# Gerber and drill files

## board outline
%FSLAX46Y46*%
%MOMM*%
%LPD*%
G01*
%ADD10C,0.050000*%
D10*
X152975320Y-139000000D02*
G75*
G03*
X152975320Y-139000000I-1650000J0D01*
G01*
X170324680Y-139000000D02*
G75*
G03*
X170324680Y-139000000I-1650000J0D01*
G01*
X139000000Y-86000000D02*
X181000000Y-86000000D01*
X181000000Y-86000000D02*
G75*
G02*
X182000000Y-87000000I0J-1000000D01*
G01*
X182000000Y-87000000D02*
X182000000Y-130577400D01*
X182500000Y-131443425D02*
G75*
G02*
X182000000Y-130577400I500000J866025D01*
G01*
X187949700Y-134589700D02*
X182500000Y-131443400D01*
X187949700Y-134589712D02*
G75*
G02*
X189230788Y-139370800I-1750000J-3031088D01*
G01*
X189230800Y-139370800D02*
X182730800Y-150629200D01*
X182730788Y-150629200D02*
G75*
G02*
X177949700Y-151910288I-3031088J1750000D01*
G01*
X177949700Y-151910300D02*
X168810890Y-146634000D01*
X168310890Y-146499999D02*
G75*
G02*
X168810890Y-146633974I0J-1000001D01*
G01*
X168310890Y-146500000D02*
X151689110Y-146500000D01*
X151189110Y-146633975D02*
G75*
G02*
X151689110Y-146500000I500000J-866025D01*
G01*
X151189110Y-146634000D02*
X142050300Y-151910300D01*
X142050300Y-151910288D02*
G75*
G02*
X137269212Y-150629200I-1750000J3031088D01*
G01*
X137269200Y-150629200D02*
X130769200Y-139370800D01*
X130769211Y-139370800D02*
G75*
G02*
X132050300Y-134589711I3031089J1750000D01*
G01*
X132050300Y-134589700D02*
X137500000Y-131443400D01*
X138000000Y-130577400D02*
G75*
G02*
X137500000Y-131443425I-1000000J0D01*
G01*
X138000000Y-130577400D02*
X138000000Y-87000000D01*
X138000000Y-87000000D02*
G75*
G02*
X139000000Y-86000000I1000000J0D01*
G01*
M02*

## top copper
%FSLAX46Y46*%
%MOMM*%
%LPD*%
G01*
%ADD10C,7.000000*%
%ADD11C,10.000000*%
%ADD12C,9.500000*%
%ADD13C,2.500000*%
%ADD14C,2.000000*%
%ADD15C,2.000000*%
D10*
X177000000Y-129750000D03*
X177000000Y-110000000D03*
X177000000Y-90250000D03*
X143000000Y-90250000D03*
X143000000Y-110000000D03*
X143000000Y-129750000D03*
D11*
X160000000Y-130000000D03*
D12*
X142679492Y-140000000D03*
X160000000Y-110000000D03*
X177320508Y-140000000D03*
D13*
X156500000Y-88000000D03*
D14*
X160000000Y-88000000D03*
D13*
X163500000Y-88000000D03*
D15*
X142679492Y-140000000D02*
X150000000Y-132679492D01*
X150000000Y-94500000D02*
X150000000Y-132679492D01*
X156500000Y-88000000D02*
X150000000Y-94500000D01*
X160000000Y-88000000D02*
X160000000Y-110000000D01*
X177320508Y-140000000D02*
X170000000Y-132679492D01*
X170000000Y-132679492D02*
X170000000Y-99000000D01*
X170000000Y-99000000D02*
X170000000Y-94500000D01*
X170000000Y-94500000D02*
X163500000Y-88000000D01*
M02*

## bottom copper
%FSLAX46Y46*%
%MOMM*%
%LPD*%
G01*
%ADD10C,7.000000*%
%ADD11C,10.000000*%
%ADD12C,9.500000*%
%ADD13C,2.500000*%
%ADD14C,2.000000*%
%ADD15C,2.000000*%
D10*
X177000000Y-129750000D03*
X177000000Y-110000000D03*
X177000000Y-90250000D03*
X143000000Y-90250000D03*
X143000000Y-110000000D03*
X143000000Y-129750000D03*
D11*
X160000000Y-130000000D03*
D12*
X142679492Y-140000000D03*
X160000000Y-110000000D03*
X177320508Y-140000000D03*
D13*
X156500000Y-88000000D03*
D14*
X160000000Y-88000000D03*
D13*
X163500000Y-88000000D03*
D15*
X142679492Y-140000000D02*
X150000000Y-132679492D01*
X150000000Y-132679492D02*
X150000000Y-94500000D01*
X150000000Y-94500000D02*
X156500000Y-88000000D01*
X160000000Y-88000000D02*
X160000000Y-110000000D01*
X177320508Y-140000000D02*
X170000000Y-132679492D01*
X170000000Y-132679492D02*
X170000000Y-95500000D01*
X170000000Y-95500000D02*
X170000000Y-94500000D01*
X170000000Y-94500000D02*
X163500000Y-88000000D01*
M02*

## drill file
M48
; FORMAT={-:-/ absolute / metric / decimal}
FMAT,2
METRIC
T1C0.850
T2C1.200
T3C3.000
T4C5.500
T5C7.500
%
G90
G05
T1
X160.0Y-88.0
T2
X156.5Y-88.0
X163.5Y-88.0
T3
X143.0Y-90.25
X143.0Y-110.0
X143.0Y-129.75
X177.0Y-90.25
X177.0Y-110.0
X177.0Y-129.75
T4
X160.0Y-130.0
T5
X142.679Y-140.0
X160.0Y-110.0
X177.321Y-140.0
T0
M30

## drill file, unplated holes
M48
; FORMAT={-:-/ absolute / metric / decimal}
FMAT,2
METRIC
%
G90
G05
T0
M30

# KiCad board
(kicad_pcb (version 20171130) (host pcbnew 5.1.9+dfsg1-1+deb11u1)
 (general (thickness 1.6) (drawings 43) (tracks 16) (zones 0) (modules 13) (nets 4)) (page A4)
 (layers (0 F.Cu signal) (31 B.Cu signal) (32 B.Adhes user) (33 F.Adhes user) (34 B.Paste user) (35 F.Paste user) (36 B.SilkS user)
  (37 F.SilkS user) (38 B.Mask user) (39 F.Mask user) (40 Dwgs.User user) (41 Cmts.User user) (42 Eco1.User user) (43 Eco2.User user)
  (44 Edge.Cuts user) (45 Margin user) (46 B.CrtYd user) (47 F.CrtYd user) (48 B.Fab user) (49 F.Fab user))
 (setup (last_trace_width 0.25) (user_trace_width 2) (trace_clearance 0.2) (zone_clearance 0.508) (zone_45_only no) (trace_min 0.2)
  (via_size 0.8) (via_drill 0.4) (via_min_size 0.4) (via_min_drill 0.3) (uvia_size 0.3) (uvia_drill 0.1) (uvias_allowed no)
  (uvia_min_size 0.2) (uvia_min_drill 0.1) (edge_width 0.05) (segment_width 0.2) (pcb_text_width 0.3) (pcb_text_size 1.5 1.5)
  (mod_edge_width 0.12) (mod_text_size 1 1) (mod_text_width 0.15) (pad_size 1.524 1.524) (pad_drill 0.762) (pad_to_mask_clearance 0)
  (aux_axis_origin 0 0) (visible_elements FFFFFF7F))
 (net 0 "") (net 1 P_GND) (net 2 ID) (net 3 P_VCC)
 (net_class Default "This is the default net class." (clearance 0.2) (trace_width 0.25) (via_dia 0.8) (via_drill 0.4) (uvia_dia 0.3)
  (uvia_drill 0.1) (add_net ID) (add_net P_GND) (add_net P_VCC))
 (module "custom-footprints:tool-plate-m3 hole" (layer F.Cu) (at 177 129.75)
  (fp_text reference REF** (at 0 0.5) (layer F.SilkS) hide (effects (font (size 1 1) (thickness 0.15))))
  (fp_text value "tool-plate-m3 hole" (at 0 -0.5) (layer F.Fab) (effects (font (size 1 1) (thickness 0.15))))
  (pad 1 thru_hole circle (at 0 0) (size 7 7) (drill 3) (layers *.Cu *.Mask)))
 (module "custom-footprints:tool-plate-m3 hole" (layer F.Cu) (at 177 110)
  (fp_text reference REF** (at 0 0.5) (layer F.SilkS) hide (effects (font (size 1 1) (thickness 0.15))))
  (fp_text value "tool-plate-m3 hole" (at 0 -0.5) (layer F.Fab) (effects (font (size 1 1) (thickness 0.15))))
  (pad 1 thru_hole circle (at 0 0) (size 7 7) (drill 3) (layers *.Cu *.Mask)))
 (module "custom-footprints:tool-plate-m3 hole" (layer F.Cu) (at 177 90.25)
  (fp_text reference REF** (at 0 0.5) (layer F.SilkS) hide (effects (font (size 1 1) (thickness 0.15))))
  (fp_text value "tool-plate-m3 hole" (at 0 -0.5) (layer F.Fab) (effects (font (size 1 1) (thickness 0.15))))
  (pad 1 thru_hole circle (at 0 0) (size 7 7) (drill 3) (layers *.Cu *.Mask)))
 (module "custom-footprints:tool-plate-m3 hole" (layer F.Cu) (at 143 90.25)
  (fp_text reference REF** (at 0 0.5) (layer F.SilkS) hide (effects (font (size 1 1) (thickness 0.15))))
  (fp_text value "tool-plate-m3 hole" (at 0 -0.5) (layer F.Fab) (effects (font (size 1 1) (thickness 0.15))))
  (pad 1 thru_hole circle (at 0 0) (size 7 7) (drill 3) (layers *.Cu *.Mask)))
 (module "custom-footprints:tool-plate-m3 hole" (layer F.Cu) (at 143 110)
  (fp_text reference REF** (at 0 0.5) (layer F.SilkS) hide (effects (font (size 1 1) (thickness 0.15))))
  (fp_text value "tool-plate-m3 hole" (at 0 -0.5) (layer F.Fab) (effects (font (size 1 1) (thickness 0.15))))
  (pad 1 thru_hole circle (at 0 0) (size 7 7) (drill 3) (layers *.Cu *.Mask)))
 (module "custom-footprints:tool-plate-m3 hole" (layer F.Cu) (at 143 129.75)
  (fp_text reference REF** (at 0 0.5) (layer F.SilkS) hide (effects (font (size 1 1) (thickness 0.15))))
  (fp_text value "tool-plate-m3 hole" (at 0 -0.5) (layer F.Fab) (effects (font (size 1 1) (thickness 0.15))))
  (pad 1 thru_hole circle (at 0 0) (size 7 7) (drill 3) (layers *.Cu *.Mask)))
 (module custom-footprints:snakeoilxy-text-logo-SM (layer B.Cu) (at 160 142 180)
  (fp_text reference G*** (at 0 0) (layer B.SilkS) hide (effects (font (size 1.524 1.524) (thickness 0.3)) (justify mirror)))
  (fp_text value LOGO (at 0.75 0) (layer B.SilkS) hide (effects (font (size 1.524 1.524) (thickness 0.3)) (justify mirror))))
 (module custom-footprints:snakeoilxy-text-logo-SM (layer F.Cu) (at 160 142)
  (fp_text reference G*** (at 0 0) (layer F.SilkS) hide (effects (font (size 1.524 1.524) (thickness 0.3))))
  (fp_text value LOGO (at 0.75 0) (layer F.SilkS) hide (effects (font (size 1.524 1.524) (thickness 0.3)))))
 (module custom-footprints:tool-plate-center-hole (layer F.Cu) (at 160 130)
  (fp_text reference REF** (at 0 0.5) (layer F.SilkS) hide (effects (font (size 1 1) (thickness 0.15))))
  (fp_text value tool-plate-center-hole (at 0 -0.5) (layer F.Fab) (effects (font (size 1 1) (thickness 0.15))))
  (pad 1 thru_hole circle (at 0 0) (size 10 10) (drill 5.5) (layers *.Cu *.Mask)))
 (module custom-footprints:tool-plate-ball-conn (layer F.Cu) (at 160 130 120)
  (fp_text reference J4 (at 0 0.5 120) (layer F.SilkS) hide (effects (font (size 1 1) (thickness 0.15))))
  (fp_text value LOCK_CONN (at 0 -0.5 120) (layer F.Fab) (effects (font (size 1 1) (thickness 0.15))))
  (pad 1 thru_hole circle (at 0 -20 120) (size 9.5 9.5) (drill 7.5) (layers *.Cu *.Mask) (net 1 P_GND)))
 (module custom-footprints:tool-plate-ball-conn (layer F.Cu) (at 160 130)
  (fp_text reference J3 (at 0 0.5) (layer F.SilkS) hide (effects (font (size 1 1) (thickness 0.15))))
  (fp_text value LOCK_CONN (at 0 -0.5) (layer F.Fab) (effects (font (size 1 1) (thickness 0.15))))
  (pad 1 thru_hole circle (at 0 -20) (size 9.5 9.5) (drill 7.5) (layers *.Cu *.Mask) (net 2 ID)))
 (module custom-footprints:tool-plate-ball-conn (layer F.Cu) (at 160 130 240)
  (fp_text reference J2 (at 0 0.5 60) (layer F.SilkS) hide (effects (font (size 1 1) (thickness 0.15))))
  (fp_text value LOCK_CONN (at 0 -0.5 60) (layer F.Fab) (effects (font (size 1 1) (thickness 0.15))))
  (pad 1 thru_hole circle (at 0 -20 240) (size 9.5 9.5) (drill 7.5) (layers *.Cu *.Mask) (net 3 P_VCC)))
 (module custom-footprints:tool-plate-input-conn (layer F.Cu) (at 160 88 180)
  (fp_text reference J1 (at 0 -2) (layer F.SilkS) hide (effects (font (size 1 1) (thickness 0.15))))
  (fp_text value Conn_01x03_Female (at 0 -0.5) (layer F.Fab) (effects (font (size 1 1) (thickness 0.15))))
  (pad 1 thru_hole circle (at 3.5 0 180) (size 2.5 2.5) (drill 1.2) (layers *.Cu *.Mask) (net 1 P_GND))
  (pad 2 thru_hole circle (at 0 0 180) (size 2 2) (drill 0.85) (layers *.Cu *.Mask) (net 2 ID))
  (pad 3 thru_hole circle (at -3.5 0 180) (size 2.5 2.5) (drill 1.2) (layers *.Cu *.Mask) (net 3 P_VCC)))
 (gr_circle (center 151.32532 139) (end 149.67532 139) (layer Edge.Cuts) (width 0.05))
 (gr_circle (center 168.67468 139) (end 167.02468 139) (layer Edge.Cuts) (width 0.05))
 (gr_line (start 139 86) (end 181 86) (layer Edge.Cuts) (width 0.05))
 (gr_arc (start 181 87) (end 182 87) (angle -90) (layer Edge.Cuts) (width 0.05))
 (gr_line (start 182 87) (end 182 130.5774) (layer Edge.Cuts) (width 0.05))
 (gr_arc (start 183 130.5774) (end 182 130.5774) (angle -60) (layer Edge.Cuts) (width 0.05))
 (gr_line (start 187.9497 134.5897) (end 182.5 131.4434) (layer Edge.Cuts) (width 0.05))
 (gr_arc (start 186.1997 137.6208) (end 189.230788 139.3708) (angle -90) (layer Edge.Cuts) (width 0.05))
 (gr_line (start 189.2308 139.3708) (end 182.7308 150.6292) (layer Edge.Cuts) (width 0.05))
 (gr_arc (start 179.6997 148.8792) (end 177.9497 151.910288) (angle -90) (layer Edge.Cuts) (width 0.05))
 (gr_line (start 177.9497 151.9103) (end 168.81089 146.634) (layer Edge.Cuts) (width 0.05))
 (gr_arc (start 168.31089 147.5) (end 168.81089 146.633974) (angle -30) (layer Edge.Cuts) (width 0.05))
 (gr_line (start 168.31089 146.5) (end 151.68911 146.5) (layer Edge.Cuts) (width 0.05))
 (gr_arc (start 151.68911 147.5) (end 151.68911 146.5) (angle -30) (layer Edge.Cuts) (width 0.05))
 (gr_line (start 151.18911 146.634) (end 142.0503 151.9103) (layer Edge.Cuts) (width 0.05))
 (gr_arc (start 140.3003 148.8792) (end 137.269212 150.6292) (angle -90) (layer Edge.Cuts) (width 0.05))
 (gr_line (start 137.2692 150.6292) (end 130.7692 139.3708) (layer Edge.Cuts) (width 0.05))
 (gr_arc (start 133.8003 137.6208) (end 132.0503 134.589711) (angle -90) (layer Edge.Cuts) (width 0.05))
 (gr_line (start 132.0503 134.5897) (end 137.5 131.4434) (layer Edge.Cuts) (width 0.05))
 (gr_arc (start 137 130.5774) (end 137.5 131.443425) (angle -60) (layer Edge.Cuts) (width 0.05))
 (gr_line (start 138 130.5774) (end 138 87) (layer Edge.Cuts) (width 0.05))
 (gr_arc (start 139 87) (end 139 86) (angle -90) (layer Edge.Cuts) (width 0.05))
 (segment (start 142.679492 140) (end 150 132.679492) (width 2) (layer F.Cu) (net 1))
 (segment (start 150 94.5) (end 150 132.679492) (width 2) (layer F.Cu) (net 1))
 (segment (start 156.5 88) (end 150 94.5) (width 2) (layer F.Cu) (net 1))
 (segment (start 142.679492 140) (end 150 132.679492) (width 2) (layer B.Cu) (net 1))
 (segment (start 150 132.679492) (end 150 94.5) (width 2) (layer B.Cu) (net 1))
 (segment (start 150 94.5) (end 156.5 88) (width 2) (layer B.Cu) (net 1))
 (segment (start 160 88) (end 160 110) (width 2) (layer B.Cu) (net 2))
 (segment (start 160 88) (end 160 110) (width 2) (layer F.Cu) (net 2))
 (segment (start 177.320508 140) (end 170 132.679492) (width 2) (layer F.Cu) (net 3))
 (segment (start 170 132.679492) (end 170 99) (width 2) (layer F.Cu) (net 3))
 (segment (start 170 99) (end 170 94.5) (width 2) (layer F.Cu) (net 3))
 (segment (start 170 94.5) (end 163.5 88) (width 2) (layer F.Cu) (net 3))
 (segment (start 177.320508 140) (end 170 132.679492) (width 2) (layer B.Cu) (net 3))
 (segment (start 170 132.679492) (end 170 95.5) (width 2) (layer B.Cu) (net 3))
 (segment (start 170 95.5) (end 170 94.5) (width 2) (layer B.Cu) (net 3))
 (segment (start 170 94.5) (end 163.5 88) (width 2) (layer B.Cu) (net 3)))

